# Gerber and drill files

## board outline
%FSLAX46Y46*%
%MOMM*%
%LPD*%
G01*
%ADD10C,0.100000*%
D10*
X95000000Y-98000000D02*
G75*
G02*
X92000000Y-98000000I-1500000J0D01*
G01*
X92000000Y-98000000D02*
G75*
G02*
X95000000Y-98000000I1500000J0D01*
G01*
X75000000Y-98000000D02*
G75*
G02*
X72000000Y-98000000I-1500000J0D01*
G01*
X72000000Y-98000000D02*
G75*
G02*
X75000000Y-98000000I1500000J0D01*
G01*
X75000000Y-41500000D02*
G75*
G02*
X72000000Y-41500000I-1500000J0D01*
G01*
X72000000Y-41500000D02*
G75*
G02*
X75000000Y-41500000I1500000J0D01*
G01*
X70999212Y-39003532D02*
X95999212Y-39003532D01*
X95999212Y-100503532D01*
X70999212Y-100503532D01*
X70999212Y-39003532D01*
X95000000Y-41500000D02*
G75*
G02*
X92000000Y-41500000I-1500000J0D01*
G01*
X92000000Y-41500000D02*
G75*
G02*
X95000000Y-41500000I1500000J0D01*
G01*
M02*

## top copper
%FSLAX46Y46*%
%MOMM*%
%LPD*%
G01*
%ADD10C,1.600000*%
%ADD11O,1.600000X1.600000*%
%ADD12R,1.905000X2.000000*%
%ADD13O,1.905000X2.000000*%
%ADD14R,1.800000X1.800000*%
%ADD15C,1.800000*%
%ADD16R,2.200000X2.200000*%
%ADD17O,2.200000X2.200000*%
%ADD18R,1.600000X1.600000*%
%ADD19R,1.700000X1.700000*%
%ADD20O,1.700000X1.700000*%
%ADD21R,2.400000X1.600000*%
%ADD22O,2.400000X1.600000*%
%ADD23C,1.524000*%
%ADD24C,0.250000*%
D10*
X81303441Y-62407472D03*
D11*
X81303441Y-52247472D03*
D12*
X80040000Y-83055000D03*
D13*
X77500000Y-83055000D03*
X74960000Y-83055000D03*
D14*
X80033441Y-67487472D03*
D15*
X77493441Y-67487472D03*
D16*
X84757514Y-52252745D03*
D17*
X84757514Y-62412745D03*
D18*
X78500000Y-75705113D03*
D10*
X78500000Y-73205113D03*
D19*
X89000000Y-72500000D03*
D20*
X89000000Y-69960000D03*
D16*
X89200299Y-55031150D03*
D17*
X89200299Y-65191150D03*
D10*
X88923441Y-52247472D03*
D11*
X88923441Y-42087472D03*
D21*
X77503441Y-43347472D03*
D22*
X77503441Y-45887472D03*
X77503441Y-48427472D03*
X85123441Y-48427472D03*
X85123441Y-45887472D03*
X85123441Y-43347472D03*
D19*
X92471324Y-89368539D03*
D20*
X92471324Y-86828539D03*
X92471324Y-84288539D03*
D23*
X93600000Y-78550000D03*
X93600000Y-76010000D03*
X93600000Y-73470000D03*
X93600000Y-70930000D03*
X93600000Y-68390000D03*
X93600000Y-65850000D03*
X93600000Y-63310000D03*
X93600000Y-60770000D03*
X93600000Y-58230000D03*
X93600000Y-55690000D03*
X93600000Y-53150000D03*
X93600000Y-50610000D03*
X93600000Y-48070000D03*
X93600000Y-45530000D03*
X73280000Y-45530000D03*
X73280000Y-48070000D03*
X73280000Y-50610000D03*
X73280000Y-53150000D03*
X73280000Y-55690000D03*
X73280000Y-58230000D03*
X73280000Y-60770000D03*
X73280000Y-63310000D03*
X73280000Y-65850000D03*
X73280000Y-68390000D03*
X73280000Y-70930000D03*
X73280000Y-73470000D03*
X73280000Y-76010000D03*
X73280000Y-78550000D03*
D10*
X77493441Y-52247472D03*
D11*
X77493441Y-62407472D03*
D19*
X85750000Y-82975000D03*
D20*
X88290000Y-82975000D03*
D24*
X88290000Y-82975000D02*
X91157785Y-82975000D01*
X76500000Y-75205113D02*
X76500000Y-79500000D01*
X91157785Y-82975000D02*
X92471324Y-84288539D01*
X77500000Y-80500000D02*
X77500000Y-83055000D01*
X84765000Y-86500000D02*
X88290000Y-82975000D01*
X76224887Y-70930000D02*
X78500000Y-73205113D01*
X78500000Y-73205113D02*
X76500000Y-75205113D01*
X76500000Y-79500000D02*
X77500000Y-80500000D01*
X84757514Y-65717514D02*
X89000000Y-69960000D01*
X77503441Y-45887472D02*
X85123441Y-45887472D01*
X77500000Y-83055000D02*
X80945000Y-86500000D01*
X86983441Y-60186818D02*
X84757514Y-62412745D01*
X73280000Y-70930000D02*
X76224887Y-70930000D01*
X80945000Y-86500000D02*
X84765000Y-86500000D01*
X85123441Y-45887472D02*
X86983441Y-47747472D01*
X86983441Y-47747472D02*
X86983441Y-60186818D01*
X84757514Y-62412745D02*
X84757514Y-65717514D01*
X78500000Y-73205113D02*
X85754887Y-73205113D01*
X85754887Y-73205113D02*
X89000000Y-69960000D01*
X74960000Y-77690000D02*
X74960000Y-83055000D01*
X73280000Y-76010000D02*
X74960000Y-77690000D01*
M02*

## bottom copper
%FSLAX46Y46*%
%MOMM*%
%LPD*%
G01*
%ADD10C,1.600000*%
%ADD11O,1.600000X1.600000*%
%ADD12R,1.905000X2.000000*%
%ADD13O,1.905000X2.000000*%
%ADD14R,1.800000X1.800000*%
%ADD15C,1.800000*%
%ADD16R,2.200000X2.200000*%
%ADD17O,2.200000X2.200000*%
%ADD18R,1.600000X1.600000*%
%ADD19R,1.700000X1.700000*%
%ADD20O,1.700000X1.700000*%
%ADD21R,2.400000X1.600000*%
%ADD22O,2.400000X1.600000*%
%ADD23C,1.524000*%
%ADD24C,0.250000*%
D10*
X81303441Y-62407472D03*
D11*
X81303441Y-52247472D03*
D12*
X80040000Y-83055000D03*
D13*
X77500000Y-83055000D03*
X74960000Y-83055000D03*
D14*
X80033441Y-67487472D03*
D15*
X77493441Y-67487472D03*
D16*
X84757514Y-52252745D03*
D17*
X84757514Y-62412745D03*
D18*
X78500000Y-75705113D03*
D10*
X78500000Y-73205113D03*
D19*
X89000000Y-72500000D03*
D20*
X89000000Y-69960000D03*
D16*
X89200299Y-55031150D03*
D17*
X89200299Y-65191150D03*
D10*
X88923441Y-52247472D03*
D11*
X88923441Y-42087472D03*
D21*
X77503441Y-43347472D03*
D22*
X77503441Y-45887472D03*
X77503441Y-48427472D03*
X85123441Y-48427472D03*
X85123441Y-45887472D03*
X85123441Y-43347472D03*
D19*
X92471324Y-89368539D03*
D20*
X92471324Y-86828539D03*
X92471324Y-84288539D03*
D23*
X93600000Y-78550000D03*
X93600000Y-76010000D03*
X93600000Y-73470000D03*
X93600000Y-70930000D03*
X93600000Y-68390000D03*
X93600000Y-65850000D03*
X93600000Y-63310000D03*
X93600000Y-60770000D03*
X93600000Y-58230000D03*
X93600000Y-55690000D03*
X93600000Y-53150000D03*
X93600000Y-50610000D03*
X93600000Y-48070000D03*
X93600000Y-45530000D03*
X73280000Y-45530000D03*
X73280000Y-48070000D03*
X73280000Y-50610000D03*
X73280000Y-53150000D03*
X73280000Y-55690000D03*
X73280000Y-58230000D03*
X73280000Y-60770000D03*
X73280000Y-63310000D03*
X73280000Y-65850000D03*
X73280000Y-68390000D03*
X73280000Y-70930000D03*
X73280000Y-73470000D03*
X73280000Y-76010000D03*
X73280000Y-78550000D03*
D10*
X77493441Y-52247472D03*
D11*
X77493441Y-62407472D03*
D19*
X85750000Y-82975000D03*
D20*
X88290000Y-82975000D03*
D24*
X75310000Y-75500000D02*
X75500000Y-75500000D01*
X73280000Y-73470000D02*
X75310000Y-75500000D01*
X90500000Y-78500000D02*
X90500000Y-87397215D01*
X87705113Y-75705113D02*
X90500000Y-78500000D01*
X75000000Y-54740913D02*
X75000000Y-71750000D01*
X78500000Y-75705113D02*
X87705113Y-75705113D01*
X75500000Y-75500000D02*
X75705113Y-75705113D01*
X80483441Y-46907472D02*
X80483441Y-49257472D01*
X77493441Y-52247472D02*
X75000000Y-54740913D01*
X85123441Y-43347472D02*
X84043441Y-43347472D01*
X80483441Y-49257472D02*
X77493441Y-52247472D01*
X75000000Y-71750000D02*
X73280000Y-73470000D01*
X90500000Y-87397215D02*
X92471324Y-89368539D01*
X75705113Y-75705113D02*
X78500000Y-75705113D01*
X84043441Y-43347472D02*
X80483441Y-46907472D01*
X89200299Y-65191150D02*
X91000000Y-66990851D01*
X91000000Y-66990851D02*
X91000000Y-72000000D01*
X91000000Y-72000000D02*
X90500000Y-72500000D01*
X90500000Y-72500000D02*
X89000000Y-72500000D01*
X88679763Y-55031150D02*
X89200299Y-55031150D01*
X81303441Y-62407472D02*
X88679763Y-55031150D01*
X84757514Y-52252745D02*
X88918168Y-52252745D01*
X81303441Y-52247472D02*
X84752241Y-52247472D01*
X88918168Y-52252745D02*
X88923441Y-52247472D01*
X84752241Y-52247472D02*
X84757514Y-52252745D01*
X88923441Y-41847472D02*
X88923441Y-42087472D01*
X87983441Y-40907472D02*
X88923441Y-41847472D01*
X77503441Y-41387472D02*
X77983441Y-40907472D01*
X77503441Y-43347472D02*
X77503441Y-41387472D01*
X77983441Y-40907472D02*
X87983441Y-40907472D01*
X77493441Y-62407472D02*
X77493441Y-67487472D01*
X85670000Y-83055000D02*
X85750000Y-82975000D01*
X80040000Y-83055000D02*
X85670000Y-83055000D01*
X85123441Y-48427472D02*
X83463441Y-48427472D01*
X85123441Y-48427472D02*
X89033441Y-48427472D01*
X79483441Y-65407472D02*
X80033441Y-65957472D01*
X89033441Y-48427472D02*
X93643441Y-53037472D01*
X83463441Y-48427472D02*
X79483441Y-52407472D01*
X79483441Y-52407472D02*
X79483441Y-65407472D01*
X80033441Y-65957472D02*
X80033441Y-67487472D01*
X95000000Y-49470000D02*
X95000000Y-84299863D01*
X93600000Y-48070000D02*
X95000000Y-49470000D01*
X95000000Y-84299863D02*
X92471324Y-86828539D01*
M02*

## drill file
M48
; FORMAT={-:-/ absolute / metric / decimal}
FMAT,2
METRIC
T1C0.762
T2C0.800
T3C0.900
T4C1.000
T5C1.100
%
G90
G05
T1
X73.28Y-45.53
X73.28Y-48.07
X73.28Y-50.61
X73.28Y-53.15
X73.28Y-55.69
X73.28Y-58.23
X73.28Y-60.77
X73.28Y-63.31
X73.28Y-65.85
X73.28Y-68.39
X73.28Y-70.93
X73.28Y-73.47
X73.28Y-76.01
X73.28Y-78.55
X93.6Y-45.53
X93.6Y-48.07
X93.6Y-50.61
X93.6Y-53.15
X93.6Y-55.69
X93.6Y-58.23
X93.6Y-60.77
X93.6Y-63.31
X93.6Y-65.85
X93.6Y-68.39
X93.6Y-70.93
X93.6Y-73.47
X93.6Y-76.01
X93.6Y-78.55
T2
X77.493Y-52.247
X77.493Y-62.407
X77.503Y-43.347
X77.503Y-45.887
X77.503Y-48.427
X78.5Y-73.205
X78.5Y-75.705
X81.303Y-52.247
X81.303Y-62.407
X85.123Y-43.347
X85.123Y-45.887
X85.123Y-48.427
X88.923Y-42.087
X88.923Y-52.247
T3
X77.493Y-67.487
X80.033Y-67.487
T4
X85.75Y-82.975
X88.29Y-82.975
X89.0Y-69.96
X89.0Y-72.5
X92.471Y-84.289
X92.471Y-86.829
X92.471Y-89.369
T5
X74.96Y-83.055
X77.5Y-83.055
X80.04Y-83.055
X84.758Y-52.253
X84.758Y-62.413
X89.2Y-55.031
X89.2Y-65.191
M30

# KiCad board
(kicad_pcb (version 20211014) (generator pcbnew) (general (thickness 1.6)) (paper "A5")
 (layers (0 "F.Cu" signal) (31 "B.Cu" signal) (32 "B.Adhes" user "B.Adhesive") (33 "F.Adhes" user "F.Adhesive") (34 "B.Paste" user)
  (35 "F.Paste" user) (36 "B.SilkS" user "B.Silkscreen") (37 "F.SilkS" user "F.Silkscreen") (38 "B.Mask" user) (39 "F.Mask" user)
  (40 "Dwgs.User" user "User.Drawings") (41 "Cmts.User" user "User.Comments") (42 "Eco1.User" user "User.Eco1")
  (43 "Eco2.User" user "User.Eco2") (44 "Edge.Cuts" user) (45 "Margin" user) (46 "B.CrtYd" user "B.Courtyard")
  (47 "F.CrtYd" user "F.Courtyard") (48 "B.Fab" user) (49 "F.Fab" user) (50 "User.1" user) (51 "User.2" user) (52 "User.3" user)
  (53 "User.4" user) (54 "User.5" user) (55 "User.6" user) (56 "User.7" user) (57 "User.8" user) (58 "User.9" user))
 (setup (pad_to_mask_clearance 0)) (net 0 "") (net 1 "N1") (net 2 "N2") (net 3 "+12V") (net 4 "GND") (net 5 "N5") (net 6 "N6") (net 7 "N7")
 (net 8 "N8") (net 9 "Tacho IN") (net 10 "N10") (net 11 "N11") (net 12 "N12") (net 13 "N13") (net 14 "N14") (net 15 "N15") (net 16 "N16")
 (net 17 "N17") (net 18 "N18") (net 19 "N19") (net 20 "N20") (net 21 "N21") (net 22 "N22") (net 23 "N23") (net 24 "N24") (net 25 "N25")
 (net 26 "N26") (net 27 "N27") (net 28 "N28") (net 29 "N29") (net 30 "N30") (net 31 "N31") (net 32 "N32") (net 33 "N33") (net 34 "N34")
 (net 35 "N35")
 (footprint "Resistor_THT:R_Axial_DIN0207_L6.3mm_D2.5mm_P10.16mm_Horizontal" (layer "F.Cu") (at 81.303441 62.407472 90)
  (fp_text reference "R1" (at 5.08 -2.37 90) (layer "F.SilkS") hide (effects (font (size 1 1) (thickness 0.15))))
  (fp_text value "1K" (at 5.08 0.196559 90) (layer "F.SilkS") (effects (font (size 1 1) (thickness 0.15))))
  (pad "1" thru_hole circle (at 0 0 90) (size 1.6 1.6) (drill 0.8) (layers *.Cu *.Mask) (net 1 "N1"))
  (pad "2" thru_hole oval (at 10.16 0 90) (size 1.6 1.6) (drill 0.8) (layers *.Cu *.Mask) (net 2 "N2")))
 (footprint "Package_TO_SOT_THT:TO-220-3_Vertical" (layer "F.Cu") (at 80.04 83.055 180)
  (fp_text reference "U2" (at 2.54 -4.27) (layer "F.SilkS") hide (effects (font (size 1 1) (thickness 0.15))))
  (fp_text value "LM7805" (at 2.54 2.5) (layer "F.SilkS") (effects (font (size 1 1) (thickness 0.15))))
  (pad "1" thru_hole rect (at 0 0 180) (size 1.905 2) (drill 1.1) (layers *.Cu *.Mask) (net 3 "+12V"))
  (pad "2" thru_hole oval (at 2.54 0 180) (size 1.905 2) (drill 1.1) (layers *.Cu *.Mask) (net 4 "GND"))
  (pad "3" thru_hole oval (at 5.08 0 180) (size 1.905 2) (drill 1.1) (layers *.Cu *.Mask) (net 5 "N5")))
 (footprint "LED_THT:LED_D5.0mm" (layer "F.Cu") (at 80.033441 67.487472 180)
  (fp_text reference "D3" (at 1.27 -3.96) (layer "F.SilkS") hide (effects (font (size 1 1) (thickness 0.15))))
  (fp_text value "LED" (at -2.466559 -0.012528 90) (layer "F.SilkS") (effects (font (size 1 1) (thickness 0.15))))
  (pad "1" thru_hole rect (at 0 0 180) (size 1.8 1.8) (drill 0.9) (layers *.Cu *.Mask) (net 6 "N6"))
  (pad "2" thru_hole circle (at 2.54 0 180) (size 1.8 1.8) (drill 0.9) (layers *.Cu *.Mask) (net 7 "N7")))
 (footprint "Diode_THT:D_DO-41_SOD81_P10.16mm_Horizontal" (layer "F.Cu") (at 84.757514 52.252745 -90)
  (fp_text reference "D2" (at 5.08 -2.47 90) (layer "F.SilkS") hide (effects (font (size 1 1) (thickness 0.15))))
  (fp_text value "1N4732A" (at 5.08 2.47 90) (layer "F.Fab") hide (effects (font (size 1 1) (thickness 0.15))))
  (pad "1" thru_hole rect (at 0 0 270) (size 2.2 2.2) (drill 1.1) (layers *.Cu *.Mask) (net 2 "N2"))
  (pad "2" thru_hole oval (at 10.16 0 270) (size 2.2 2.2) (drill 1.1) (layers *.Cu *.Mask) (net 4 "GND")))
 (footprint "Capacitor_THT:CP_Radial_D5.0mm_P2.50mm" (layer "F.Cu") (at 78.5 75.705113 90)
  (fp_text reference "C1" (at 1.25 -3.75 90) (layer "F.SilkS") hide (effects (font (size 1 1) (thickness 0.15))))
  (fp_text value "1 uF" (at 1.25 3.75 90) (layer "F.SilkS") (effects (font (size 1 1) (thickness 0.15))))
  (pad "1" thru_hole rect (at 0 0 90) (size 1.6 1.6) (drill 0.8) (layers *.Cu *.Mask) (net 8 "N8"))
  (pad "2" thru_hole circle (at 2.5 0 90) (size 1.6 1.6) (drill 0.8) (layers *.Cu *.Mask) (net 4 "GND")))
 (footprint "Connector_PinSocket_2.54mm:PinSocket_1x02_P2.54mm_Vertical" (layer "F.Cu") (at 89 72.5 180)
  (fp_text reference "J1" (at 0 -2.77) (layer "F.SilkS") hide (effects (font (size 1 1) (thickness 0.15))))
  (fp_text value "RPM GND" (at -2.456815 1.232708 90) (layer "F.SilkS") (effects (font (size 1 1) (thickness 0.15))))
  (pad "1" thru_hole rect (at 0 0 180) (size 1.7 1.7) (drill 1) (layers *.Cu *.Mask) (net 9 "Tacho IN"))
  (pad "2" thru_hole oval (at 0 2.54 180) (size 1.7 1.7) (drill 1) (layers *.Cu *.Mask) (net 4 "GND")))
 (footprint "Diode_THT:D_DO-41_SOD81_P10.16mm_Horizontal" (layer "F.Cu") (at 89.200299 55.03115 -90)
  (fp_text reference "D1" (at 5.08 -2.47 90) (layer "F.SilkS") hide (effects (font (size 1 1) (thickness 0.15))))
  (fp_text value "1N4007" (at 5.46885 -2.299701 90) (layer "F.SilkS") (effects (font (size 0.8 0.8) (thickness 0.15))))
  (pad "1" thru_hole rect (at 0 0 270) (size 2.2 2.2) (drill 1.1) (layers *.Cu *.Mask) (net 1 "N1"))
  (pad "2" thru_hole oval (at 10.16 0 270) (size 2.2 2.2) (drill 1.1) (layers *.Cu *.Mask) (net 9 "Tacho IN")))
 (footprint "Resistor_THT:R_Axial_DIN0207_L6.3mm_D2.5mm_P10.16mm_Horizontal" (layer "F.Cu") (at 88.923441 52.247472 90)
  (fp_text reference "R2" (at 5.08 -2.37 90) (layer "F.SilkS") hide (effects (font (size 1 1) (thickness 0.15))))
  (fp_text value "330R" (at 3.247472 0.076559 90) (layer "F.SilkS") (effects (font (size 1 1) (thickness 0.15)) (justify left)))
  (pad "1" thru_hole circle (at 0 0 90) (size 1.6 1.6) (drill 0.8) (layers *.Cu *.Mask) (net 2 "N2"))
  (pad "2" thru_hole oval (at 10.16 0 90) (size 1.6 1.6) (drill 0.8) (layers *.Cu *.Mask) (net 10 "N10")))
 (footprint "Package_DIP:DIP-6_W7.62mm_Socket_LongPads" (layer "F.Cu") (at 77.503441 43.347472)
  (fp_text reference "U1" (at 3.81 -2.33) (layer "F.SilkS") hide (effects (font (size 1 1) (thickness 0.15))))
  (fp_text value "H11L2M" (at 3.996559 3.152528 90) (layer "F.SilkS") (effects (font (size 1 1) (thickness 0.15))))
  (pad "1" thru_hole rect (at 0 0) (size 2.4 1.6) (drill 0.8) (layers *.Cu *.Mask) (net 10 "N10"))
  (pad "2" thru_hole oval (at 0 2.54) (size 2.4 1.6) (drill 0.8) (layers *.Cu *.Mask) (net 4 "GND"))
  (pad "3" thru_hole oval (at 0 5.08) (size 2.4 1.6) (drill 0.8) (layers *.Cu *.Mask) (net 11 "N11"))
  (pad "4" thru_hole oval (at 7.62 5.08) (size 2.4 1.6) (drill 0.8) (layers *.Cu *.Mask) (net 6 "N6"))
  (pad "5" thru_hole oval (at 7.62 2.54) (size 2.4 1.6) (drill 0.8) (layers *.Cu *.Mask) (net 4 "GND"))
  (pad "6" thru_hole oval (at 7.62 0) (size 2.4 1.6) (drill 0.8) (layers *.Cu *.Mask) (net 8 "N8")))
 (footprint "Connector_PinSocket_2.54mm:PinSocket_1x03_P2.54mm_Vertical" (layer "F.Cu") (at 92.471324 89.368539 180)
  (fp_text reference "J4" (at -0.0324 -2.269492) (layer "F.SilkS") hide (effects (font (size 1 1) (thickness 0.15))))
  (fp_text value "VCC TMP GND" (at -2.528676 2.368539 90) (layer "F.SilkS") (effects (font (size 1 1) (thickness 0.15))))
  (pad "1" thru_hole rect (at 0 0 180) (size 1.7 1.7) (drill 1) (layers *.Cu *.Mask) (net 8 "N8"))
  (pad "2" thru_hole oval (at 0 2.54 180) (size 1.7 1.7) (drill 1) (layers *.Cu *.Mask) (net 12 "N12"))
  (pad "3" thru_hole oval (at 0 5.08 180) (size 1.7 1.7) (drill 1) (layers *.Cu *.Mask) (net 4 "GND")))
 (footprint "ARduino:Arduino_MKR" (layer "F.Cu") (at 96.14 78.55 180)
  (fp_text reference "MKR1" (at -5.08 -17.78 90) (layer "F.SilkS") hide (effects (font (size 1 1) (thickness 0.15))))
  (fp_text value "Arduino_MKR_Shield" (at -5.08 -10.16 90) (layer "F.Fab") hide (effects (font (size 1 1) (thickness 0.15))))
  (pad "1" thru_hole circle locked (at 2.54 0 180) (size 1.524 1.524) (drill 0.762) (layers *.Cu *.Mask) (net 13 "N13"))
  (pad "2" thru_hole circle locked (at 2.54 2.54 180) (size 1.524 1.524) (drill 0.762) (layers *.Cu *.Mask) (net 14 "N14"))
  (pad "3" thru_hole circle locked (at 2.54 5.08 180) (size 1.524 1.524) (drill 0.762) (layers *.Cu *.Mask) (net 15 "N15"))
  (pad "4" thru_hole circle locked (at 2.54 7.62 180) (size 1.524 1.524) (drill 0.762) (layers *.Cu *.Mask) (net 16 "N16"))
  (pad "5" thru_hole circle locked (at 2.54 10.16 180) (size 1.524 1.524) (drill 0.762) (layers *.Cu *.Mask) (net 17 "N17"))
  (pad "6" thru_hole circle locked (at 2.54 12.7 180) (size 1.524 1.524) (drill 0.762) (layers *.Cu *.Mask) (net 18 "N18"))
  (pad "7" thru_hole circle locked (at 2.54 15.24 180) (size 1.524 1.524) (drill 0.762) (layers *.Cu *.Mask) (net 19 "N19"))
  (pad "8" thru_hole circle locked (at 2.54 17.78 180) (size 1.524 1.524) (drill 0.762) (layers *.Cu *.Mask) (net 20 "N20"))
  (pad "9" thru_hole circle locked (at 2.54 20.32 180) (size 1.524 1.524) (drill 0.762) (layers *.Cu *.Mask) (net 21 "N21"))
  (pad "10" thru_hole circle locked (at 2.54 22.86 180) (size 1.524 1.524) (drill 0.762) (layers *.Cu *.Mask) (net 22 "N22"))
  (pad "11" thru_hole circle locked (at 2.54 25.4 180) (size 1.524 1.524) (drill 0.762) (layers *.Cu *.Mask) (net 6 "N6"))
  (pad "12" thru_hole circle locked (at 2.54 27.94 180) (size 1.524 1.524) (drill 0.762) (layers *.Cu *.Mask) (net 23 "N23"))
  (pad "13" thru_hole circle locked (at 2.54 30.48 180) (size 1.524 1.524) (drill 0.762) (layers *.Cu *.Mask) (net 12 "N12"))
  (pad "14" thru_hole circle locked (at 2.54 33.02 180) (size 1.524 1.524) (drill 0.762) (layers *.Cu *.Mask) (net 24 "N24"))
  (pad "15" thru_hole circle locked (at 22.86 33.02 180) (size 1.524 1.524) (drill 0.762) (layers *.Cu *.Mask) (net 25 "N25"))
  (pad "16" thru_hole circle locked (at 22.86 30.48 180) (size 1.524 1.524) (drill 0.762) (layers *.Cu *.Mask) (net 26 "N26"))
  (pad "17" thru_hole circle locked (at 22.86 27.94 180) (size 1.524 1.524) (drill 0.762) (layers *.Cu *.Mask) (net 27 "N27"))
  (pad "18" thru_hole circle locked (at 22.86 25.4 180) (size 1.524 1.524) (drill 0.762) (layers *.Cu *.Mask) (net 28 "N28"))
  (pad "19" thru_hole circle locked (at 22.86 22.86 180) (size 1.524 1.524) (drill 0.762) (layers *.Cu *.Mask) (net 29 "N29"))
  (pad "20" thru_hole circle locked (at 22.86 20.32 180) (size 1.524 1.524) (drill 0.762) (layers *.Cu *.Mask) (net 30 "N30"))
  (pad "21" thru_hole circle locked (at 22.86 17.78 180) (size 1.524 1.524) (drill 0.762) (layers *.Cu *.Mask) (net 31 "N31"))
  (pad "22" thru_hole circle locked (at 22.86 15.24 180) (size 1.524 1.524) (drill 0.762) (layers *.Cu *.Mask) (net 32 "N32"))
  (pad "23" thru_hole circle locked (at 22.86 12.7 180) (size 1.524 1.524) (drill 0.762) (layers *.Cu *.Mask) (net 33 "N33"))
  (pad "24" thru_hole circle locked (at 22.86 10.16 180) (size 1.524 1.524) (drill 0.762) (layers *.Cu *.Mask) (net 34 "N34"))
  (pad "25" thru_hole circle locked (at 22.86 7.62 180) (size 1.524 1.524) (drill 0.762) (layers *.Cu *.Mask) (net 4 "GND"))
  (pad "26" thru_hole circle locked (at 22.86 5.08 180) (size 1.524 1.524) (drill 0.762) (layers *.Cu *.Mask) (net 8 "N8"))
  (pad "27" thru_hole circle locked (at 22.86 2.54 180) (size 1.524 1.524) (drill 0.762) (layers *.Cu *.Mask) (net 5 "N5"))
  (pad "28" thru_hole circle locked (at 22.86 0 180) (size 1.524 1.524) (drill 0.762) (layers *.Cu *.Mask) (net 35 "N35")))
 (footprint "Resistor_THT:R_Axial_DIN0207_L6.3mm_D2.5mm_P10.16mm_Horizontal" (layer "F.Cu") (at 77.493441 52.247472 -90)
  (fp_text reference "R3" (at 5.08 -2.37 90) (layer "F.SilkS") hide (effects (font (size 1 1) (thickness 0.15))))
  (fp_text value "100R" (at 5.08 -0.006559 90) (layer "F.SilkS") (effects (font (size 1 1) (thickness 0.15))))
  (pad "1" thru_hole circle (at 0 0 270) (size 1.6 1.6) (drill 0.8) (layers *.Cu *.Mask) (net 8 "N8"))
  (pad "2" thru_hole oval (at 10.16 0 270) (size 1.6 1.6) (drill 0.8) (layers *.Cu *.Mask) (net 7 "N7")))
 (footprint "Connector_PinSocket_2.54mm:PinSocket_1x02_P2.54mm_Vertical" (layer "F.Cu") (at 85.75 82.975 90)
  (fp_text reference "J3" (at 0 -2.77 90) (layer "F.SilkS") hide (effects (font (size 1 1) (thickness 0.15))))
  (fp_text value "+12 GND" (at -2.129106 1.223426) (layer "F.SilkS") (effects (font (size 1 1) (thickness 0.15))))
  (pad "1" thru_hole rect (at 0 0 90) (size 1.7 1.7) (drill 1) (layers *.Cu *.Mask) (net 3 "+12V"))
  (pad "2" thru_hole oval (at 0 2.54 90) (size 1.7 1.7) (drill 1) (layers *.Cu *.Mask) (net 4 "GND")))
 (gr_circle (center 93.5 98) (end 95 98) (layer "Edge.Cuts") (width 0.1) (fill none))
 (gr_circle (center 73.5 98) (end 75 98) (layer "Edge.Cuts") (width 0.1) (fill none))
 (gr_circle (center 73.5 41.5) (end 75 41.5) (layer "Edge.Cuts") (width 0.1) (fill none))
 (gr_rect (start 70.999212 39.003532) (end 95.999212 100.503532) (layer "Edge.Cuts") (width 0.1) (fill none))
 (gr_circle (center 93.5 41.5) (end 95 41.5) (layer "Edge.Cuts") (width 0.1) (fill none))
 (segment (start 75.31 75.5) (end 75.5 75.5) (width 0.25) (layer "B.Cu") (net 8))
 (segment (start 73.28 73.47) (end 75.31 75.5) (width 0.25) (layer "B.Cu") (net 8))
 (segment (start 90.5 78.5) (end 90.5 87.397215) (width 0.25) (layer "B.Cu") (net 8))
 (segment (start 87.705113 75.705113) (end 90.5 78.5) (width 0.25) (layer "B.Cu") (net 8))
 (segment (start 75 54.740913) (end 75 71.75) (width 0.25) (layer "B.Cu") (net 8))
 (segment (start 78.5 75.705113) (end 87.705113 75.705113) (width 0.25) (layer "B.Cu") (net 8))
 (segment (start 75.5 75.5) (end 75.705113 75.705113) (width 0.25) (layer "B.Cu") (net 8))
 (segment (start 80.483441 46.907472) (end 80.483441 49.257472) (width 0.25) (layer "B.Cu") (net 8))
 (segment (start 77.493441 52.247472) (end 75 54.740913) (width 0.25) (layer "B.Cu") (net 8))
 (segment (start 85.123441 43.347472) (end 84.043441 43.347472) (width 0.25) (layer "B.Cu") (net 8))
 (segment (start 80.483441 49.257472) (end 77.493441 52.247472) (width 0.25) (layer "B.Cu") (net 8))
 (segment (start 75 71.75) (end 73.28 73.47) (width 0.25) (layer "B.Cu") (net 8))
 (segment (start 90.5 87.397215) (end 92.471324 89.368539) (width 0.25) (layer "B.Cu") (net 8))
 (segment (start 75.705113 75.705113) (end 78.5 75.705113) (width 0.25) (layer "B.Cu") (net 8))
 (segment (start 84.043441 43.347472) (end 80.483441 46.907472) (width 0.25) (layer "B.Cu") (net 8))
 (segment (start 89.200299 65.19115) (end 91 66.990851) (width 0.25) (layer "B.Cu") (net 9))
 (segment (start 91 66.990851) (end 91 72) (width 0.25) (layer "B.Cu") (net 9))
 (segment (start 91 72) (end 90.5 72.5) (width 0.25) (layer "B.Cu") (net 9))
 (segment (start 90.5 72.5) (end 89 72.5) (width 0.25) (layer "B.Cu") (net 9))
 (segment (start 88.679763 55.03115) (end 89.200299 55.03115) (width 0.25) (layer "B.Cu") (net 1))
 (segment (start 81.303441 62.407472) (end 88.679763 55.03115) (width 0.25) (layer "B.Cu") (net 1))
 (segment (start 88.29 82.975) (end 91.157785 82.975) (width 0.25) (layer "F.Cu") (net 4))
 (segment (start 76.5 75.205113) (end 76.5 79.5) (width 0.25) (layer "F.Cu") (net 4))
 (segment (start 91.157785 82.975) (end 92.471324 84.288539) (width 0.25) (layer "F.Cu") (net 4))
 (segment (start 77.5 80.5) (end 77.5 83.055) (width 0.25) (layer "F.Cu") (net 4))
 (segment (start 84.765 86.5) (end 88.29 82.975) (width 0.25) (layer "F.Cu") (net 4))
 (segment (start 76.224887 70.93) (end 78.5 73.205113) (width 0.25) (layer "F.Cu") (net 4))
 (segment (start 78.5 73.205113) (end 76.5 75.205113) (width 0.25) (layer "F.Cu") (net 4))
 (segment (start 76.5 79.5) (end 77.5 80.5) (width 0.25) (layer "F.Cu") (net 4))
 (segment (start 84.757514 65.717514) (end 89 69.96) (width 0.25) (layer "F.Cu") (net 4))
 (segment (start 77.503441 45.887472) (end 85.123441 45.887472) (width 0.25) (layer "F.Cu") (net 4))
 (segment (start 77.5 83.055) (end 80.945 86.5) (width 0.25) (layer "F.Cu") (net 4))
 (segment (start 86.983441 60.186818) (end 84.757514 62.412745) (width 0.25) (layer "F.Cu") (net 4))
 (segment (start 73.28 70.93) (end 76.224887 70.93) (width 0.25) (layer "F.Cu") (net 4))
 (segment (start 80.945 86.5) (end 84.765 86.5) (width 0.25) (layer "F.Cu") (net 4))
 (segment (start 85.123441 45.887472) (end 86.983441 47.747472) (width 0.25) (layer "F.Cu") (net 4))
 (segment (start 86.983441 47.747472) (end 86.983441 60.186818) (width 0.25) (layer "F.Cu") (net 4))
 (segment (start 84.757514 62.412745) (end 84.757514 65.717514) (width 0.25) (layer "F.Cu") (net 4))
 (segment (start 78.5 73.205113) (end 85.754887 73.205113) (width 0.25) (layer "F.Cu") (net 4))
 (segment (start 85.754887 73.205113) (end 89 69.96) (width 0.25) (layer "F.Cu") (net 4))
 (segment (start 84.757514 52.252745) (end 88.918168 52.252745) (width 0.25) (layer "B.Cu") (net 2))
 (segment (start 81.303441 52.247472) (end 84.752241 52.247472) (width 0.25) (layer "B.Cu") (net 2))
 (segment (start 88.918168 52.252745) (end 88.923441 52.247472) (width 0.25) (layer "B.Cu") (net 2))
 (segment (start 84.752241 52.247472) (end 84.757514 52.252745) (width 0.25) (layer "B.Cu") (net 2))
 (segment (start 88.923441 41.847472) (end 88.923441 42.087472) (width 0.25) (layer "B.Cu") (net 10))
 (segment (start 87.983441 40.907472) (end 88.923441 41.847472) (width 0.25) (layer "B.Cu") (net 10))
 (segment (start 77.503441 41.387472) (end 77.983441 40.907472) (width 0.25) (layer "B.Cu") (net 10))
 (segment (start 77.503441 43.347472) (end 77.503441 41.387472) (width 0.25) (layer "B.Cu") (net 10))
 (segment (start 77.983441 40.907472) (end 87.983441 40.907472) (width 0.25) (layer "B.Cu") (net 10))
 (segment (start 77.493441 62.407472) (end 77.493441 67.487472) (width 0.25) (layer "B.Cu") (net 7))
 (segment (start 85.67 83.055) (end 85.75 82.975) (width 0.25) (layer "B.Cu") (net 3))
 (segment (start 80.04 83.055) (end 85.67 83.055) (width 0.25) (layer "B.Cu") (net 3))
 (segment (start 85.123441 48.427472) (end 83.463441 48.427472) (width 0.25) (layer "B.Cu") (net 6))
 (segment (start 85.123441 48.427472) (end 89.033441 48.427472) (width 0.25) (layer "B.Cu") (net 6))
 (segment (start 79.483441 65.407472) (end 80.033441 65.957472) (width 0.25) (layer "B.Cu") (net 6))
 (segment (start 89.033441 48.427472) (end 93.643441 53.037472) (width 0.25) (layer "B.Cu") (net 6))
 (segment (start 83.463441 48.427472) (end 79.483441 52.407472) (width 0.25) (layer "B.Cu") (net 6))
 (segment (start 79.483441 52.407472) (end 79.483441 65.407472) (width 0.25) (layer "B.Cu") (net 6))
 (segment (start 80.033441 65.957472) (end 80.033441 67.487472) (width 0.25) (layer "B.Cu") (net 6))
 (segment (start 74.96 77.69) (end 74.96 83.055) (width 0.25) (layer "F.Cu") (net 5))
 (segment (start 73.28 76.01) (end 74.96 77.69) (width 0.25) (layer "F.Cu") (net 5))
 (segment (start 95 49.47) (end 95 84.299863) (width 0.25) (layer "B.Cu") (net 12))
 (segment (start 93.6 48.07) (end 95 49.47) (width 0.25) (layer "B.Cu") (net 12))
 (segment (start 95 84.299863) (end 92.471324 86.828539) (width 0.25) (layer "B.Cu") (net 12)))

